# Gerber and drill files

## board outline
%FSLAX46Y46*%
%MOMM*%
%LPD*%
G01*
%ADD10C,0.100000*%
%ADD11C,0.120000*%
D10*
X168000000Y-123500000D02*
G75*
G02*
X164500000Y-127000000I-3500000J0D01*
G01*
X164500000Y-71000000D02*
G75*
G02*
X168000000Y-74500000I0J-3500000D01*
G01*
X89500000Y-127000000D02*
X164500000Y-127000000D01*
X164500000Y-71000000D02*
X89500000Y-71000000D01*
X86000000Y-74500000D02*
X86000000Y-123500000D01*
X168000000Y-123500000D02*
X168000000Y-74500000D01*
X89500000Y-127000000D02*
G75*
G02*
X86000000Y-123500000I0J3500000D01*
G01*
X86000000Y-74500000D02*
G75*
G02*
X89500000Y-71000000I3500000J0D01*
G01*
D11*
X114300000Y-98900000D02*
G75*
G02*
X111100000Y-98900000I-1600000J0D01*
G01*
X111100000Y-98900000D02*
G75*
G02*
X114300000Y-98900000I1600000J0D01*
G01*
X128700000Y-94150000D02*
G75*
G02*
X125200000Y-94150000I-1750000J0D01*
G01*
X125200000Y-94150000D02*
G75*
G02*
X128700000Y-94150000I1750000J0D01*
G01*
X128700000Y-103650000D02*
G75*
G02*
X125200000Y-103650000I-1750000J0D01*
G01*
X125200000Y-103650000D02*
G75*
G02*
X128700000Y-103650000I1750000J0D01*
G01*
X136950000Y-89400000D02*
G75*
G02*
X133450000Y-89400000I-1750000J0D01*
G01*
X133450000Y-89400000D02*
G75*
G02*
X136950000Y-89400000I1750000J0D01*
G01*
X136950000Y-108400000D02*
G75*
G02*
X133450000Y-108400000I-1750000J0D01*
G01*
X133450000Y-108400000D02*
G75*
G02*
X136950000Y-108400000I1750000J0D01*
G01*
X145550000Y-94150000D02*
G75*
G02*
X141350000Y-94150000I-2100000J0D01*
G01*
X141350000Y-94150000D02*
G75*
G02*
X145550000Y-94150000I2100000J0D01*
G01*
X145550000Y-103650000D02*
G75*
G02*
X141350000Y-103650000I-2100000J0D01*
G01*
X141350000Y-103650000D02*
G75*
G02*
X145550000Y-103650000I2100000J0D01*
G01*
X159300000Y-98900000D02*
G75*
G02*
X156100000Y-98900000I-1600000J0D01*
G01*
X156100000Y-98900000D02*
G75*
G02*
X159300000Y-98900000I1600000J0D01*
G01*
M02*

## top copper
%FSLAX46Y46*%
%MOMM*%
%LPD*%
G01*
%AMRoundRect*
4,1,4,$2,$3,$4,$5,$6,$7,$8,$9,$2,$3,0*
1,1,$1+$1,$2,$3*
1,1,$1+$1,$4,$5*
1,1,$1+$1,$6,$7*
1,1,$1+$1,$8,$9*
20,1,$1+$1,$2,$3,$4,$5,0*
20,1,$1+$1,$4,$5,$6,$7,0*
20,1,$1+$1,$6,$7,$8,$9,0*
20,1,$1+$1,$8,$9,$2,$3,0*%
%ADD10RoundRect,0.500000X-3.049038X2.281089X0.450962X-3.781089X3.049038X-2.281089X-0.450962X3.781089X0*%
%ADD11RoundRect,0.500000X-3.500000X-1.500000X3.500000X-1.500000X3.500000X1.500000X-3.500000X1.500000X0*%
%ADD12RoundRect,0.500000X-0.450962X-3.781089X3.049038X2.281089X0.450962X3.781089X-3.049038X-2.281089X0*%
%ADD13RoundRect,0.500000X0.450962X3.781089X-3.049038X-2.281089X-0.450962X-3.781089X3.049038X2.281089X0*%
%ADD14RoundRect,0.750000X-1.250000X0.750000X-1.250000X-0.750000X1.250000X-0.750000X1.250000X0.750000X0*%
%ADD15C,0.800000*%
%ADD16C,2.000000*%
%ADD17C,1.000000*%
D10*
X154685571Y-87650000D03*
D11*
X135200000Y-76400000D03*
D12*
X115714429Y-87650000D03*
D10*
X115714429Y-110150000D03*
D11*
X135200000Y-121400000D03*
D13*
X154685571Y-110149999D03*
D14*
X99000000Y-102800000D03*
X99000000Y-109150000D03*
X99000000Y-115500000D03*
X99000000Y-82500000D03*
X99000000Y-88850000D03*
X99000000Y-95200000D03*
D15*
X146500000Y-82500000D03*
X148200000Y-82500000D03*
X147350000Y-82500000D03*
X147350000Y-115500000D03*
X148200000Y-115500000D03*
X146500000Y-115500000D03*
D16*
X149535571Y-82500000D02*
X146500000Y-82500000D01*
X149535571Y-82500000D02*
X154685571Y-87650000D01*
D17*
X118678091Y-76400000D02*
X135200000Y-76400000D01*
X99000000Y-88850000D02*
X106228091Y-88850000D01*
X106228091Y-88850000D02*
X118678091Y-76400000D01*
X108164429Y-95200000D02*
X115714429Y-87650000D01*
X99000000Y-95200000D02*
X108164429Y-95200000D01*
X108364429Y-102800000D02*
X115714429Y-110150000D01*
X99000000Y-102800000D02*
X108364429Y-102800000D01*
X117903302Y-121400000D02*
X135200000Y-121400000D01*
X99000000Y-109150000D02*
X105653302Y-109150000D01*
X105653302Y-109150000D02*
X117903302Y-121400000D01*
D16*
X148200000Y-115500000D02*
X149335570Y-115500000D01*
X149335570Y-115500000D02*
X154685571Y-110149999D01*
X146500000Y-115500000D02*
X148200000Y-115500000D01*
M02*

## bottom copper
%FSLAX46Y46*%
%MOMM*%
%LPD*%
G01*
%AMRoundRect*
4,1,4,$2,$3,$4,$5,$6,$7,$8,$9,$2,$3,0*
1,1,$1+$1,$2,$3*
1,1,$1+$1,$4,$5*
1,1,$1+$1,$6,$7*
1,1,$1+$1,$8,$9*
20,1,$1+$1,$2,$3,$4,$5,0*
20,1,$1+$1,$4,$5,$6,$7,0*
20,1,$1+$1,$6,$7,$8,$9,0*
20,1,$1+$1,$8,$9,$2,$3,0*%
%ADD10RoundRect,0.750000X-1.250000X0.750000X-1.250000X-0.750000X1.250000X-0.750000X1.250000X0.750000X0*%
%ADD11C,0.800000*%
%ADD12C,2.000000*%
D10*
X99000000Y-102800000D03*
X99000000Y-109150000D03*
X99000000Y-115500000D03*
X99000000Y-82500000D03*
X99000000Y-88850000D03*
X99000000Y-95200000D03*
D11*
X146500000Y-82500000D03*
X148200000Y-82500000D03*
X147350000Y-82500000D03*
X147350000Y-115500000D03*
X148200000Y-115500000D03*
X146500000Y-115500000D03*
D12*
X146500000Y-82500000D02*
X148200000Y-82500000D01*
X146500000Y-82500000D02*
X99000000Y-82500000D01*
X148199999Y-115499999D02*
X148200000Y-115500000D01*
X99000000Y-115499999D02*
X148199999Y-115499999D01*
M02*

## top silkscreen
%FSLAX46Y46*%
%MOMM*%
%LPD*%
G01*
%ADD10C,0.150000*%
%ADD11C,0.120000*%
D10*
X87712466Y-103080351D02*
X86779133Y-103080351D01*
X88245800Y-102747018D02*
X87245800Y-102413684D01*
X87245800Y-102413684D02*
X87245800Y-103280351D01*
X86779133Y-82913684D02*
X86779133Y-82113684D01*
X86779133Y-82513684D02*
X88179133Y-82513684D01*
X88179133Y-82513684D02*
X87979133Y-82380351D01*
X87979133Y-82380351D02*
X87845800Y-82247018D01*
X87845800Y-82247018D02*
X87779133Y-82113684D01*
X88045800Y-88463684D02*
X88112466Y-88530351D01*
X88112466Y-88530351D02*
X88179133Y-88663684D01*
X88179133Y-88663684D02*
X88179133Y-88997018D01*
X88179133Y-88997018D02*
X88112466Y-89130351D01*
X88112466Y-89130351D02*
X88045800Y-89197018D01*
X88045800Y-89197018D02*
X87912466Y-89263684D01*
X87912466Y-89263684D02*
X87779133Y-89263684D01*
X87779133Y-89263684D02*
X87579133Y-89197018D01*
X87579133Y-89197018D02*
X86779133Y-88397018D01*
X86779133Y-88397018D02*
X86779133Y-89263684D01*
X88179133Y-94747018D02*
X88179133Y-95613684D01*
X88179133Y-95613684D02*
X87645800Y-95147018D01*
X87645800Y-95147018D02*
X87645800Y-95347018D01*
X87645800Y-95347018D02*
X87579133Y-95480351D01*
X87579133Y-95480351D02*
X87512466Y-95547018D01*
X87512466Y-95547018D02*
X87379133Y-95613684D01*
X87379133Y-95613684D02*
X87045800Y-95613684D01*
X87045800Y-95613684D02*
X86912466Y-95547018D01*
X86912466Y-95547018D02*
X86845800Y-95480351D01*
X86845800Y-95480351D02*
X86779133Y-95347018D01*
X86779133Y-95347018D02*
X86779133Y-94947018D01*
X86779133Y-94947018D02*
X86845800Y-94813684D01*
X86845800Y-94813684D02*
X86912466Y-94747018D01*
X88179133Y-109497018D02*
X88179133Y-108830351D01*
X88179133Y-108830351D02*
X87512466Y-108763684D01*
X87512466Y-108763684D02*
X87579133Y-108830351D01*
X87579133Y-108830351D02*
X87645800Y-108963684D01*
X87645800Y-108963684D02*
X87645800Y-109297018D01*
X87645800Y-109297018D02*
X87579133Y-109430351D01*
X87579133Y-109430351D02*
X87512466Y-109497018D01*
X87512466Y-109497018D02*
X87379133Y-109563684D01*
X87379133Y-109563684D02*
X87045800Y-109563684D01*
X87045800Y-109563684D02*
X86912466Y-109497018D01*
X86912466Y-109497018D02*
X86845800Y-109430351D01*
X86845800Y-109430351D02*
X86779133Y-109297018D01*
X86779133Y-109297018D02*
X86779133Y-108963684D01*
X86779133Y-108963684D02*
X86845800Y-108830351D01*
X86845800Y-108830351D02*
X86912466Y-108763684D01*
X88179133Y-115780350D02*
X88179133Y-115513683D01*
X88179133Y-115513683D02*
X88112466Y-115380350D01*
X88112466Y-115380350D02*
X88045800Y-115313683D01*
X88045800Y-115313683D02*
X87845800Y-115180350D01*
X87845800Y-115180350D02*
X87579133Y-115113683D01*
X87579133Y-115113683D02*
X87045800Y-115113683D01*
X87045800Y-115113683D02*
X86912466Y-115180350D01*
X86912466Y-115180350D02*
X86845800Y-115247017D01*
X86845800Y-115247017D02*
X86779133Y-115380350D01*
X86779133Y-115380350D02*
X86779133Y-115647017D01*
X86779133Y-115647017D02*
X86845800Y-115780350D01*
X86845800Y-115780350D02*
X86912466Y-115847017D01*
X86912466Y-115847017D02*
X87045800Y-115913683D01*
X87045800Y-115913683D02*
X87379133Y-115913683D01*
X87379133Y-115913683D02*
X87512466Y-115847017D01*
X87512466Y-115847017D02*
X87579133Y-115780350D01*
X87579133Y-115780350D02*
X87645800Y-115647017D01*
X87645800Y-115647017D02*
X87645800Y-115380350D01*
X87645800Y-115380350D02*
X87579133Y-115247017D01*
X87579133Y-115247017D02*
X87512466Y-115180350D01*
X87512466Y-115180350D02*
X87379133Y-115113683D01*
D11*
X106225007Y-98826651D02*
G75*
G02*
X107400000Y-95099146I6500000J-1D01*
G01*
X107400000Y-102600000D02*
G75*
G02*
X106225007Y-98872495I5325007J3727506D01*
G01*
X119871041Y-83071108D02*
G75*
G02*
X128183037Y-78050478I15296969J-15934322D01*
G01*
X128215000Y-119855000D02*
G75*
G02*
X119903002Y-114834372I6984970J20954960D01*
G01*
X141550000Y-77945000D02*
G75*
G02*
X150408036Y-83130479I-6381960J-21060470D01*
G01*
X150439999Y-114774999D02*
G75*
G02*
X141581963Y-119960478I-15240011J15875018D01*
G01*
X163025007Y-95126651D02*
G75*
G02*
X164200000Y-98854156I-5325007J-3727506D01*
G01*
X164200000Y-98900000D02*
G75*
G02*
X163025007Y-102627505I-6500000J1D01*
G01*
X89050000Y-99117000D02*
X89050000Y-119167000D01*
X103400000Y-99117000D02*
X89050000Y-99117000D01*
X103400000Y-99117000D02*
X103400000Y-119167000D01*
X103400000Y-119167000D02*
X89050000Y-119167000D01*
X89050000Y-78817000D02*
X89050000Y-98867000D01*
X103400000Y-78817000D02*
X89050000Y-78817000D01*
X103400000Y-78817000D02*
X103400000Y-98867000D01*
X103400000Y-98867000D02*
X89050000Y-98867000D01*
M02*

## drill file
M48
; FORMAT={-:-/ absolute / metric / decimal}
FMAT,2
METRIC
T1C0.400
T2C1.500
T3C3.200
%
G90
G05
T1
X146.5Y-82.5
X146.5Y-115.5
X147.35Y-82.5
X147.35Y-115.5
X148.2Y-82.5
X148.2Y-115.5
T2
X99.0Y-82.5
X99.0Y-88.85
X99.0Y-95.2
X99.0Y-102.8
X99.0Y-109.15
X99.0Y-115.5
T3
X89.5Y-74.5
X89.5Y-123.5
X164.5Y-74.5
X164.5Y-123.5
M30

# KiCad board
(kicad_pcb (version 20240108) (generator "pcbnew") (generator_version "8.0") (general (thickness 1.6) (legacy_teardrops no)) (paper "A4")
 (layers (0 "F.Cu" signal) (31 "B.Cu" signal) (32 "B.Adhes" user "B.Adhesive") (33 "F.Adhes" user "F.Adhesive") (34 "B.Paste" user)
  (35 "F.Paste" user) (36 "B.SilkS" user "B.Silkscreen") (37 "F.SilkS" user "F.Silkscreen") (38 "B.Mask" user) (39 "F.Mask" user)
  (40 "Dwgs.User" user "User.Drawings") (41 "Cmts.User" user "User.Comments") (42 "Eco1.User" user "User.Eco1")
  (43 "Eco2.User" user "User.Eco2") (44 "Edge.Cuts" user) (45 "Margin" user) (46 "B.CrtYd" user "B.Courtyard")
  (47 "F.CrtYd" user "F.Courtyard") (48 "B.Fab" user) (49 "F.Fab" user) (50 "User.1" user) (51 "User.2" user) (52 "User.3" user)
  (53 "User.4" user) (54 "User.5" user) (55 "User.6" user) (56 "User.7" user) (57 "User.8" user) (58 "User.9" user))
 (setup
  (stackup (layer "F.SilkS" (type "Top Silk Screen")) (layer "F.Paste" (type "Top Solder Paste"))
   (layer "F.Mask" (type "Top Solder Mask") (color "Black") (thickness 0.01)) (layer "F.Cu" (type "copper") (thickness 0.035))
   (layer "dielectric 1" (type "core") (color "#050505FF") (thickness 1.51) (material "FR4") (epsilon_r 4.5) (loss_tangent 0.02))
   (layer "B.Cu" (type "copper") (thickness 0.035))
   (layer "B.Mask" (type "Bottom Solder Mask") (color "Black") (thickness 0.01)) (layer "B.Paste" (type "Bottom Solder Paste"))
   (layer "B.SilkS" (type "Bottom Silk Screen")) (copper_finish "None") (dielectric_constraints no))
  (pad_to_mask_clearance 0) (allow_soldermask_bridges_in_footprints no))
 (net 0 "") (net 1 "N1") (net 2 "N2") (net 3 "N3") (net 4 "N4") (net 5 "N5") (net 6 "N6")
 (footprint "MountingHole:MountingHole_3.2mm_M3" (layer "F.Cu") (at 89.5 123.5)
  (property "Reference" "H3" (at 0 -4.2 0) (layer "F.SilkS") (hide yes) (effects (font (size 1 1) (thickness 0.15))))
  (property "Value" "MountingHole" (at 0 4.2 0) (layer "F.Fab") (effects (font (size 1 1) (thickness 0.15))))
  (pad "" np_thru_hole circle (at 0 0) (size 3.2 3.2) (drill 3.2) (layers "*.Cu" "*.Mask")))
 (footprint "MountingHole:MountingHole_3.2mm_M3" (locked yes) (layer "F.Cu") (at 164.5 123.5)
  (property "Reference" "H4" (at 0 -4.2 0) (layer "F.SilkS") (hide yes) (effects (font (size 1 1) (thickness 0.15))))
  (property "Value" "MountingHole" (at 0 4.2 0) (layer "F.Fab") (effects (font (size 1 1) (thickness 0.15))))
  (pad "" np_thru_hole circle (at 0 0) (size 3.2 3.2) (drill 3.2) (layers "*.Cu" "*.Mask")))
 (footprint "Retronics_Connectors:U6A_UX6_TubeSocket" (layer "F.Cu") (at 135.2 98.9 -90)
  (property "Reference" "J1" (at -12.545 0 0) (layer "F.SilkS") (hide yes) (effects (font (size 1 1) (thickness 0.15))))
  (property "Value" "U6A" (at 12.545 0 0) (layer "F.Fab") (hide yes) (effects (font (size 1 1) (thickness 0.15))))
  (fp_arc (start -0.073349 28.974993) (mid -2.027505 28.674289) (end -3.800854 27.8) (stroke (width 0.12) (type default)) (layer "F.SilkS"))
  (fp_arc (start 3.7 27.8) (mid 1.926651 28.674289) (end -0.027505 28.974993) (stroke (width 0.12) (type default)) (layer "F.SilkS"))
  (fp_arc (start -15.828892 15.328959) (mid -18.801631 11.452275) (end -20.849522 7.016963) (stroke (width 0.12) (type default))
   (layer "F.SilkS"))
  (fp_arc (start 20.955 6.985) (mid 18.907109 11.420312) (end 15.93437 15.296996) (stroke (width 0.12) (type default)) (layer "F.SilkS"))
  (fp_arc (start -20.955 -6.35) (mid -18.88593 -11.085573) (end -15.769521 -15.208036) (stroke (width 0.12) (type default))
   (layer "F.SilkS"))
  (fp_arc (start 15.874999 -15.239999) (mid 18.991407 -11.117536) (end 21.060478 -6.381963) (stroke (width 0.12) (type default))
   (layer "F.SilkS"))
  (fp_arc (start -3.773349 -27.825007) (mid -2 -28.699296) (end -0.045844 -29) (stroke (width 0.12) (type default)) (layer "F.SilkS"))
  (fp_arc (start 0 -29) (mid 1.954156 -28.699296) (end 3.727505 -27.825007) (stroke (width 0.12) (type default)) (layer "F.SilkS"))
  (fp_circle (center 0 22.5) (end 1.6 22.5) (stroke (width 0.12) (type default)) (fill none) (layer "Edge.Cuts"))
  (fp_circle (center -4.75 8.25) (end -3 8.25) (stroke (width 0.12) (type default)) (fill none) (layer "Edge.Cuts"))
  (fp_circle (center 4.75 8.25) (end 6.5 8.25) (stroke (width 0.12) (type default)) (fill none) (layer "Edge.Cuts"))
  (fp_circle (center -9.5 0) (end -7.75 0) (stroke (width 0.12) (type default)) (fill none) (layer "Edge.Cuts"))
  (fp_circle (center 9.5 0) (end 11.25 0) (stroke (width 0.12) (type default)) (fill none) (layer "Edge.Cuts"))
  (fp_circle (center -4.75 -8.25) (end -2.65 -8.25) (stroke (width 0.12) (type default)) (fill none) (layer "Edge.Cuts"))
  (fp_circle (center 4.75 -8.25) (end 6.85 -8.25) (stroke (width 0.12) (type default)) (fill none) (layer "Edge.Cuts"))
  (fp_circle (center 0 -22.5) (end 1.6 -22.5) (stroke (width 0.12) (type default)) (fill none) (layer "Edge.Cuts"))
  (pad "1" smd roundrect (at -11.25 -19.485571 300) (size 8 4) (layers "F.Cu" "F.Paste" "F.Mask") (roundrect_rratio 0.125) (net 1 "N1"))
  (pad "2" smd roundrect (at -22.5 0) (size 8 4) (layers "F.Cu" "F.Paste" "F.Mask") (roundrect_rratio 0.125) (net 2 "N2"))
  (pad "3" smd roundrect (at -11.25 19.485571 60) (size 8 4) (layers "F.Cu" "F.Paste" "F.Mask") (roundrect_rratio 0.125) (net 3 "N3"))
  (pad "4" smd roundrect (at 11.25 19.485571 300) (size 8 4) (layers "F.Cu" "F.Paste" "F.Mask") (roundrect_rratio 0.125) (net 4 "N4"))
  (pad "5" smd roundrect (at 22.5 0) (size 8 4) (layers "F.Cu" "F.Paste" "F.Mask") (roundrect_rratio 0.125) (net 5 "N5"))
  (pad "6" smd roundrect (at 11.249999 -19.485571 240) (size 8 4) (layers "F.Cu" "F.Paste" "F.Mask") (roundrect_rratio 0.125) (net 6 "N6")))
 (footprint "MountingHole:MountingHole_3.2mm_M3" (layer "F.Cu") (at 89.5 74.5)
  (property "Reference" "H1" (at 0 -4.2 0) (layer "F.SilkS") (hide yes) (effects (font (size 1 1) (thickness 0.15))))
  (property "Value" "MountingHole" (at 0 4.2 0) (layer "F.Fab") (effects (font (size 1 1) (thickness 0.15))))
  (pad "" np_thru_hole circle (at 0 0) (size 3.2 3.2) (drill 3.2) (layers "*.Cu" "*.Mask")))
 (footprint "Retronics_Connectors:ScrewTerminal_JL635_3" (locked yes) (layer "F.Cu") (at 99 102.8 -90)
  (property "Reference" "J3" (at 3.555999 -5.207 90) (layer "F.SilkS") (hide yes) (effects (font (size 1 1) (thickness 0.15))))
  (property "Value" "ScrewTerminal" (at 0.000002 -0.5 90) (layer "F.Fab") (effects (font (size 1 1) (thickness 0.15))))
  (fp_line (start -3.683 9.95) (end 16.367 9.95) (stroke (width 0.12) (type solid)) (layer "F.SilkS"))
  (fp_line (start -3.683 -4.4) (end -3.683 9.95) (stroke (width 0.12) (type solid)) (layer "F.SilkS"))
  (fp_line (start -3.683 -4.4) (end 16.367 -4.4) (stroke (width 0.12) (type solid)) (layer "F.SilkS"))
  (fp_line (start 16.367 -4.4) (end 16.367 9.95) (stroke (width 0.12) (type solid)) (layer "F.SilkS"))
  (pad "1" thru_hole roundrect (at 0 0 270) (size 3 4) (drill 1.5) (layers "*.Cu" "*.Mask") (remove_unused_layers no)
   (roundrect_rratio 0.25) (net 4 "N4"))
  (pad "2" thru_hole roundrect (at 6.35 0 270) (size 3 4) (drill 1.5) (layers "*.Cu" "*.Mask") (remove_unused_layers no)
   (roundrect_rratio 0.25) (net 5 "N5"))
  (pad "3" thru_hole roundrect (at 12.7 0 270) (size 3 4) (drill 1.5) (layers "*.Cu" "*.Mask") (remove_unused_layers no)
   (roundrect_rratio 0.25) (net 6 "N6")))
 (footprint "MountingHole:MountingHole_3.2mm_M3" (layer "F.Cu") (at 164.5 74.5)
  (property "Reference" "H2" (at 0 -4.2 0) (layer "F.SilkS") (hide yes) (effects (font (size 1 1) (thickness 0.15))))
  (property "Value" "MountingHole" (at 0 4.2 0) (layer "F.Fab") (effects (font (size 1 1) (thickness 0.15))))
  (pad "" np_thru_hole circle (at 0 0) (size 3.2 3.2) (drill 3.2) (layers "*.Cu" "*.Mask")))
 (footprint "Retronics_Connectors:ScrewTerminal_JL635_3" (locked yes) (layer "F.Cu") (at 99 82.5 -90)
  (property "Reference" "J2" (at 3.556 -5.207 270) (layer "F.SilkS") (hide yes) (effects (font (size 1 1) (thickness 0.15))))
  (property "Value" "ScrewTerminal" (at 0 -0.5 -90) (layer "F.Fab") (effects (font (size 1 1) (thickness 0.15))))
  (fp_line (start -3.683 9.95) (end 16.367 9.95) (stroke (width 0.12) (type solid)) (layer "F.SilkS"))
  (fp_line (start -3.683 -4.4) (end -3.683 9.95) (stroke (width 0.12) (type solid)) (layer "F.SilkS"))
  (fp_line (start -3.683 -4.4) (end 16.367 -4.4) (stroke (width 0.12) (type solid)) (layer "F.SilkS"))
  (fp_line (start 16.367 -4.4) (end 16.367 9.95) (stroke (width 0.12) (type solid)) (layer "F.SilkS"))
  (pad "1" thru_hole roundrect (at 0 0 270) (size 3 4) (drill 1.5) (layers "*.Cu" "*.Mask") (remove_unused_layers no)
   (roundrect_rratio 0.25) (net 1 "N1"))
  (pad "2" thru_hole roundrect (at 6.35 0 270) (size 3 4) (drill 1.5) (layers "*.Cu" "*.Mask") (remove_unused_layers no)
   (roundrect_rratio 0.25) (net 2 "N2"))
  (pad "3" thru_hole roundrect (at 12.7 0 270) (size 3 4) (drill 1.5) (layers "*.Cu" "*.Mask") (remove_unused_layers no)
   (roundrect_rratio 0.25) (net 3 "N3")))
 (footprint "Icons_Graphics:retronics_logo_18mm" (layer "B.Cu") (at 117.5 99 -90)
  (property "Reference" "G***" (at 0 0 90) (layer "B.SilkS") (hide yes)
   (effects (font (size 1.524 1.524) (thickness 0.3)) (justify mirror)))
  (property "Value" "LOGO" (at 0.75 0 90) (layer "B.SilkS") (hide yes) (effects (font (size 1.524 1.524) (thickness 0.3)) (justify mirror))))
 (gr_arc (start 168 123.5) (mid 166.974874 125.974874) (end 164.5 127) (stroke (width 0.1) (type default)) (layer "Edge.Cuts"))
 (gr_arc (start 164.5 71) (mid 166.974874 72.025126) (end 168 74.5) (stroke (width 0.1) (type default)) (layer "Edge.Cuts"))
 (gr_line (start 89.5 127) (end 164.5 127) (stroke (width 0.1) (type default)) (layer "Edge.Cuts"))
 (gr_line (start 164.5 71) (end 89.5 71) (stroke (width 0.1) (type default)) (layer "Edge.Cuts"))
 (gr_line (start 86 74.5) (end 86 123.5) (stroke (width 0.1) (type default)) (layer "Edge.Cuts"))
 (gr_line (start 168 123.5) (end 168 74.5) (stroke (width 0.1) (type default)) (layer "Edge.Cuts"))
 (gr_arc (start 89.5 127) (mid 87.025126 125.974874) (end 86 123.5) (stroke (width 0.1) (type default)) (layer "Edge.Cuts"))
 (gr_arc (start 86 74.5) (mid 87.025126 72.025126) (end 89.5 71) (stroke (width 0.1) (type default)) (layer "Edge.Cuts"))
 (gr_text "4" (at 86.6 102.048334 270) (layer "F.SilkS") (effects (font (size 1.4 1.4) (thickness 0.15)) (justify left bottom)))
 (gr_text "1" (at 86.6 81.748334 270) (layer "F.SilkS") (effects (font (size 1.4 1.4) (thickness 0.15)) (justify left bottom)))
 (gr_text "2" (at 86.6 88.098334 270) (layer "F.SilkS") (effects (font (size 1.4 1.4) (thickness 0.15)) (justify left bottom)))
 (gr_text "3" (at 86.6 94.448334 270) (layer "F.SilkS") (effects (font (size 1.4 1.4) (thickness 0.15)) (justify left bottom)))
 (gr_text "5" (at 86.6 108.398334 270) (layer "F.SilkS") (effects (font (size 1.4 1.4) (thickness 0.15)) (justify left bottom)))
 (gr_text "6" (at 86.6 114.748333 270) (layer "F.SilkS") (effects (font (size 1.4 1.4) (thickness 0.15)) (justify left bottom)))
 (segment (start 149.535571 82.5) (end 146.5 82.5) (width 2) (layer "F.Cu") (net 1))
 (segment (start 149.535571 82.5) (end 154.685571 87.65) (width 2) (layer "F.Cu") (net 1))
 (via (at 146.5 82.5) (size 0.8) (drill 0.4) (layers "F.Cu" "B.Cu") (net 1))
 (via (at 148.2 82.5) (size 0.8) (drill 0.4) (layers "F.Cu" "B.Cu") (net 1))
 (via (at 147.35 82.5) (size 0.8) (drill 0.4) (layers "F.Cu" "B.Cu") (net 1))
 (segment (start 146.5 82.5) (end 148.2 82.5) (width 2) (layer "B.Cu") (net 1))
 (segment (start 146.5 82.5) (end 99 82.5) (width 2) (layer "B.Cu") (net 1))
 (segment (start 118.678091 76.4) (end 135.2 76.4) (width 1) (layer "F.Cu") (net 2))
 (segment (start 99 88.85) (end 106.228091 88.85) (width 1) (layer "F.Cu") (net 2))
 (segment (start 106.228091 88.85) (end 118.678091 76.4) (width 1) (layer "F.Cu") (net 2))
 (segment (start 108.164429 95.2) (end 115.714429 87.65) (width 1) (layer "F.Cu") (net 3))
 (segment (start 99 95.2) (end 108.164429 95.2) (width 1) (layer "F.Cu") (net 3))
 (segment (start 108.364429 102.8) (end 115.714429 110.15) (width 1) (layer "F.Cu") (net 4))
 (segment (start 99 102.8) (end 108.364429 102.8) (width 1) (layer "F.Cu") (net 4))
 (segment (start 117.903302 121.4) (end 135.2 121.4) (width 1) (layer "F.Cu") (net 5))
 (segment (start 99 109.15) (end 105.653302 109.15) (width 1) (layer "F.Cu") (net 5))
 (segment (start 105.653302 109.15) (end 117.903302 121.4) (width 1) (layer "F.Cu") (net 5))
 (segment (start 148.2 115.5) (end 149.33557 115.5) (width 2) (layer "F.Cu") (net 6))
 (segment (start 149.33557 115.5) (end 154.685571 110.149999) (width 2) (layer "F.Cu") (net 6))
 (segment (start 146.5 115.5) (end 148.2 115.5) (width 2) (layer "F.Cu") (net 6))
 (via (at 147.35 115.5) (size 0.8) (drill 0.4) (layers "F.Cu" "B.Cu") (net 6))
 (via (at 148.2 115.5) (size 0.8) (drill 0.4) (layers "F.Cu" "B.Cu") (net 6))
 (via (at 146.5 115.5) (size 0.8) (drill 0.4) (layers "F.Cu" "B.Cu") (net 6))
 (segment (start 148.199999 115.499999) (end 148.2 115.5) (width 2) (layer "B.Cu") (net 6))
 (segment (start 99 115.499999) (end 148.199999 115.499999) (width 2) (layer "B.Cu") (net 6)))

